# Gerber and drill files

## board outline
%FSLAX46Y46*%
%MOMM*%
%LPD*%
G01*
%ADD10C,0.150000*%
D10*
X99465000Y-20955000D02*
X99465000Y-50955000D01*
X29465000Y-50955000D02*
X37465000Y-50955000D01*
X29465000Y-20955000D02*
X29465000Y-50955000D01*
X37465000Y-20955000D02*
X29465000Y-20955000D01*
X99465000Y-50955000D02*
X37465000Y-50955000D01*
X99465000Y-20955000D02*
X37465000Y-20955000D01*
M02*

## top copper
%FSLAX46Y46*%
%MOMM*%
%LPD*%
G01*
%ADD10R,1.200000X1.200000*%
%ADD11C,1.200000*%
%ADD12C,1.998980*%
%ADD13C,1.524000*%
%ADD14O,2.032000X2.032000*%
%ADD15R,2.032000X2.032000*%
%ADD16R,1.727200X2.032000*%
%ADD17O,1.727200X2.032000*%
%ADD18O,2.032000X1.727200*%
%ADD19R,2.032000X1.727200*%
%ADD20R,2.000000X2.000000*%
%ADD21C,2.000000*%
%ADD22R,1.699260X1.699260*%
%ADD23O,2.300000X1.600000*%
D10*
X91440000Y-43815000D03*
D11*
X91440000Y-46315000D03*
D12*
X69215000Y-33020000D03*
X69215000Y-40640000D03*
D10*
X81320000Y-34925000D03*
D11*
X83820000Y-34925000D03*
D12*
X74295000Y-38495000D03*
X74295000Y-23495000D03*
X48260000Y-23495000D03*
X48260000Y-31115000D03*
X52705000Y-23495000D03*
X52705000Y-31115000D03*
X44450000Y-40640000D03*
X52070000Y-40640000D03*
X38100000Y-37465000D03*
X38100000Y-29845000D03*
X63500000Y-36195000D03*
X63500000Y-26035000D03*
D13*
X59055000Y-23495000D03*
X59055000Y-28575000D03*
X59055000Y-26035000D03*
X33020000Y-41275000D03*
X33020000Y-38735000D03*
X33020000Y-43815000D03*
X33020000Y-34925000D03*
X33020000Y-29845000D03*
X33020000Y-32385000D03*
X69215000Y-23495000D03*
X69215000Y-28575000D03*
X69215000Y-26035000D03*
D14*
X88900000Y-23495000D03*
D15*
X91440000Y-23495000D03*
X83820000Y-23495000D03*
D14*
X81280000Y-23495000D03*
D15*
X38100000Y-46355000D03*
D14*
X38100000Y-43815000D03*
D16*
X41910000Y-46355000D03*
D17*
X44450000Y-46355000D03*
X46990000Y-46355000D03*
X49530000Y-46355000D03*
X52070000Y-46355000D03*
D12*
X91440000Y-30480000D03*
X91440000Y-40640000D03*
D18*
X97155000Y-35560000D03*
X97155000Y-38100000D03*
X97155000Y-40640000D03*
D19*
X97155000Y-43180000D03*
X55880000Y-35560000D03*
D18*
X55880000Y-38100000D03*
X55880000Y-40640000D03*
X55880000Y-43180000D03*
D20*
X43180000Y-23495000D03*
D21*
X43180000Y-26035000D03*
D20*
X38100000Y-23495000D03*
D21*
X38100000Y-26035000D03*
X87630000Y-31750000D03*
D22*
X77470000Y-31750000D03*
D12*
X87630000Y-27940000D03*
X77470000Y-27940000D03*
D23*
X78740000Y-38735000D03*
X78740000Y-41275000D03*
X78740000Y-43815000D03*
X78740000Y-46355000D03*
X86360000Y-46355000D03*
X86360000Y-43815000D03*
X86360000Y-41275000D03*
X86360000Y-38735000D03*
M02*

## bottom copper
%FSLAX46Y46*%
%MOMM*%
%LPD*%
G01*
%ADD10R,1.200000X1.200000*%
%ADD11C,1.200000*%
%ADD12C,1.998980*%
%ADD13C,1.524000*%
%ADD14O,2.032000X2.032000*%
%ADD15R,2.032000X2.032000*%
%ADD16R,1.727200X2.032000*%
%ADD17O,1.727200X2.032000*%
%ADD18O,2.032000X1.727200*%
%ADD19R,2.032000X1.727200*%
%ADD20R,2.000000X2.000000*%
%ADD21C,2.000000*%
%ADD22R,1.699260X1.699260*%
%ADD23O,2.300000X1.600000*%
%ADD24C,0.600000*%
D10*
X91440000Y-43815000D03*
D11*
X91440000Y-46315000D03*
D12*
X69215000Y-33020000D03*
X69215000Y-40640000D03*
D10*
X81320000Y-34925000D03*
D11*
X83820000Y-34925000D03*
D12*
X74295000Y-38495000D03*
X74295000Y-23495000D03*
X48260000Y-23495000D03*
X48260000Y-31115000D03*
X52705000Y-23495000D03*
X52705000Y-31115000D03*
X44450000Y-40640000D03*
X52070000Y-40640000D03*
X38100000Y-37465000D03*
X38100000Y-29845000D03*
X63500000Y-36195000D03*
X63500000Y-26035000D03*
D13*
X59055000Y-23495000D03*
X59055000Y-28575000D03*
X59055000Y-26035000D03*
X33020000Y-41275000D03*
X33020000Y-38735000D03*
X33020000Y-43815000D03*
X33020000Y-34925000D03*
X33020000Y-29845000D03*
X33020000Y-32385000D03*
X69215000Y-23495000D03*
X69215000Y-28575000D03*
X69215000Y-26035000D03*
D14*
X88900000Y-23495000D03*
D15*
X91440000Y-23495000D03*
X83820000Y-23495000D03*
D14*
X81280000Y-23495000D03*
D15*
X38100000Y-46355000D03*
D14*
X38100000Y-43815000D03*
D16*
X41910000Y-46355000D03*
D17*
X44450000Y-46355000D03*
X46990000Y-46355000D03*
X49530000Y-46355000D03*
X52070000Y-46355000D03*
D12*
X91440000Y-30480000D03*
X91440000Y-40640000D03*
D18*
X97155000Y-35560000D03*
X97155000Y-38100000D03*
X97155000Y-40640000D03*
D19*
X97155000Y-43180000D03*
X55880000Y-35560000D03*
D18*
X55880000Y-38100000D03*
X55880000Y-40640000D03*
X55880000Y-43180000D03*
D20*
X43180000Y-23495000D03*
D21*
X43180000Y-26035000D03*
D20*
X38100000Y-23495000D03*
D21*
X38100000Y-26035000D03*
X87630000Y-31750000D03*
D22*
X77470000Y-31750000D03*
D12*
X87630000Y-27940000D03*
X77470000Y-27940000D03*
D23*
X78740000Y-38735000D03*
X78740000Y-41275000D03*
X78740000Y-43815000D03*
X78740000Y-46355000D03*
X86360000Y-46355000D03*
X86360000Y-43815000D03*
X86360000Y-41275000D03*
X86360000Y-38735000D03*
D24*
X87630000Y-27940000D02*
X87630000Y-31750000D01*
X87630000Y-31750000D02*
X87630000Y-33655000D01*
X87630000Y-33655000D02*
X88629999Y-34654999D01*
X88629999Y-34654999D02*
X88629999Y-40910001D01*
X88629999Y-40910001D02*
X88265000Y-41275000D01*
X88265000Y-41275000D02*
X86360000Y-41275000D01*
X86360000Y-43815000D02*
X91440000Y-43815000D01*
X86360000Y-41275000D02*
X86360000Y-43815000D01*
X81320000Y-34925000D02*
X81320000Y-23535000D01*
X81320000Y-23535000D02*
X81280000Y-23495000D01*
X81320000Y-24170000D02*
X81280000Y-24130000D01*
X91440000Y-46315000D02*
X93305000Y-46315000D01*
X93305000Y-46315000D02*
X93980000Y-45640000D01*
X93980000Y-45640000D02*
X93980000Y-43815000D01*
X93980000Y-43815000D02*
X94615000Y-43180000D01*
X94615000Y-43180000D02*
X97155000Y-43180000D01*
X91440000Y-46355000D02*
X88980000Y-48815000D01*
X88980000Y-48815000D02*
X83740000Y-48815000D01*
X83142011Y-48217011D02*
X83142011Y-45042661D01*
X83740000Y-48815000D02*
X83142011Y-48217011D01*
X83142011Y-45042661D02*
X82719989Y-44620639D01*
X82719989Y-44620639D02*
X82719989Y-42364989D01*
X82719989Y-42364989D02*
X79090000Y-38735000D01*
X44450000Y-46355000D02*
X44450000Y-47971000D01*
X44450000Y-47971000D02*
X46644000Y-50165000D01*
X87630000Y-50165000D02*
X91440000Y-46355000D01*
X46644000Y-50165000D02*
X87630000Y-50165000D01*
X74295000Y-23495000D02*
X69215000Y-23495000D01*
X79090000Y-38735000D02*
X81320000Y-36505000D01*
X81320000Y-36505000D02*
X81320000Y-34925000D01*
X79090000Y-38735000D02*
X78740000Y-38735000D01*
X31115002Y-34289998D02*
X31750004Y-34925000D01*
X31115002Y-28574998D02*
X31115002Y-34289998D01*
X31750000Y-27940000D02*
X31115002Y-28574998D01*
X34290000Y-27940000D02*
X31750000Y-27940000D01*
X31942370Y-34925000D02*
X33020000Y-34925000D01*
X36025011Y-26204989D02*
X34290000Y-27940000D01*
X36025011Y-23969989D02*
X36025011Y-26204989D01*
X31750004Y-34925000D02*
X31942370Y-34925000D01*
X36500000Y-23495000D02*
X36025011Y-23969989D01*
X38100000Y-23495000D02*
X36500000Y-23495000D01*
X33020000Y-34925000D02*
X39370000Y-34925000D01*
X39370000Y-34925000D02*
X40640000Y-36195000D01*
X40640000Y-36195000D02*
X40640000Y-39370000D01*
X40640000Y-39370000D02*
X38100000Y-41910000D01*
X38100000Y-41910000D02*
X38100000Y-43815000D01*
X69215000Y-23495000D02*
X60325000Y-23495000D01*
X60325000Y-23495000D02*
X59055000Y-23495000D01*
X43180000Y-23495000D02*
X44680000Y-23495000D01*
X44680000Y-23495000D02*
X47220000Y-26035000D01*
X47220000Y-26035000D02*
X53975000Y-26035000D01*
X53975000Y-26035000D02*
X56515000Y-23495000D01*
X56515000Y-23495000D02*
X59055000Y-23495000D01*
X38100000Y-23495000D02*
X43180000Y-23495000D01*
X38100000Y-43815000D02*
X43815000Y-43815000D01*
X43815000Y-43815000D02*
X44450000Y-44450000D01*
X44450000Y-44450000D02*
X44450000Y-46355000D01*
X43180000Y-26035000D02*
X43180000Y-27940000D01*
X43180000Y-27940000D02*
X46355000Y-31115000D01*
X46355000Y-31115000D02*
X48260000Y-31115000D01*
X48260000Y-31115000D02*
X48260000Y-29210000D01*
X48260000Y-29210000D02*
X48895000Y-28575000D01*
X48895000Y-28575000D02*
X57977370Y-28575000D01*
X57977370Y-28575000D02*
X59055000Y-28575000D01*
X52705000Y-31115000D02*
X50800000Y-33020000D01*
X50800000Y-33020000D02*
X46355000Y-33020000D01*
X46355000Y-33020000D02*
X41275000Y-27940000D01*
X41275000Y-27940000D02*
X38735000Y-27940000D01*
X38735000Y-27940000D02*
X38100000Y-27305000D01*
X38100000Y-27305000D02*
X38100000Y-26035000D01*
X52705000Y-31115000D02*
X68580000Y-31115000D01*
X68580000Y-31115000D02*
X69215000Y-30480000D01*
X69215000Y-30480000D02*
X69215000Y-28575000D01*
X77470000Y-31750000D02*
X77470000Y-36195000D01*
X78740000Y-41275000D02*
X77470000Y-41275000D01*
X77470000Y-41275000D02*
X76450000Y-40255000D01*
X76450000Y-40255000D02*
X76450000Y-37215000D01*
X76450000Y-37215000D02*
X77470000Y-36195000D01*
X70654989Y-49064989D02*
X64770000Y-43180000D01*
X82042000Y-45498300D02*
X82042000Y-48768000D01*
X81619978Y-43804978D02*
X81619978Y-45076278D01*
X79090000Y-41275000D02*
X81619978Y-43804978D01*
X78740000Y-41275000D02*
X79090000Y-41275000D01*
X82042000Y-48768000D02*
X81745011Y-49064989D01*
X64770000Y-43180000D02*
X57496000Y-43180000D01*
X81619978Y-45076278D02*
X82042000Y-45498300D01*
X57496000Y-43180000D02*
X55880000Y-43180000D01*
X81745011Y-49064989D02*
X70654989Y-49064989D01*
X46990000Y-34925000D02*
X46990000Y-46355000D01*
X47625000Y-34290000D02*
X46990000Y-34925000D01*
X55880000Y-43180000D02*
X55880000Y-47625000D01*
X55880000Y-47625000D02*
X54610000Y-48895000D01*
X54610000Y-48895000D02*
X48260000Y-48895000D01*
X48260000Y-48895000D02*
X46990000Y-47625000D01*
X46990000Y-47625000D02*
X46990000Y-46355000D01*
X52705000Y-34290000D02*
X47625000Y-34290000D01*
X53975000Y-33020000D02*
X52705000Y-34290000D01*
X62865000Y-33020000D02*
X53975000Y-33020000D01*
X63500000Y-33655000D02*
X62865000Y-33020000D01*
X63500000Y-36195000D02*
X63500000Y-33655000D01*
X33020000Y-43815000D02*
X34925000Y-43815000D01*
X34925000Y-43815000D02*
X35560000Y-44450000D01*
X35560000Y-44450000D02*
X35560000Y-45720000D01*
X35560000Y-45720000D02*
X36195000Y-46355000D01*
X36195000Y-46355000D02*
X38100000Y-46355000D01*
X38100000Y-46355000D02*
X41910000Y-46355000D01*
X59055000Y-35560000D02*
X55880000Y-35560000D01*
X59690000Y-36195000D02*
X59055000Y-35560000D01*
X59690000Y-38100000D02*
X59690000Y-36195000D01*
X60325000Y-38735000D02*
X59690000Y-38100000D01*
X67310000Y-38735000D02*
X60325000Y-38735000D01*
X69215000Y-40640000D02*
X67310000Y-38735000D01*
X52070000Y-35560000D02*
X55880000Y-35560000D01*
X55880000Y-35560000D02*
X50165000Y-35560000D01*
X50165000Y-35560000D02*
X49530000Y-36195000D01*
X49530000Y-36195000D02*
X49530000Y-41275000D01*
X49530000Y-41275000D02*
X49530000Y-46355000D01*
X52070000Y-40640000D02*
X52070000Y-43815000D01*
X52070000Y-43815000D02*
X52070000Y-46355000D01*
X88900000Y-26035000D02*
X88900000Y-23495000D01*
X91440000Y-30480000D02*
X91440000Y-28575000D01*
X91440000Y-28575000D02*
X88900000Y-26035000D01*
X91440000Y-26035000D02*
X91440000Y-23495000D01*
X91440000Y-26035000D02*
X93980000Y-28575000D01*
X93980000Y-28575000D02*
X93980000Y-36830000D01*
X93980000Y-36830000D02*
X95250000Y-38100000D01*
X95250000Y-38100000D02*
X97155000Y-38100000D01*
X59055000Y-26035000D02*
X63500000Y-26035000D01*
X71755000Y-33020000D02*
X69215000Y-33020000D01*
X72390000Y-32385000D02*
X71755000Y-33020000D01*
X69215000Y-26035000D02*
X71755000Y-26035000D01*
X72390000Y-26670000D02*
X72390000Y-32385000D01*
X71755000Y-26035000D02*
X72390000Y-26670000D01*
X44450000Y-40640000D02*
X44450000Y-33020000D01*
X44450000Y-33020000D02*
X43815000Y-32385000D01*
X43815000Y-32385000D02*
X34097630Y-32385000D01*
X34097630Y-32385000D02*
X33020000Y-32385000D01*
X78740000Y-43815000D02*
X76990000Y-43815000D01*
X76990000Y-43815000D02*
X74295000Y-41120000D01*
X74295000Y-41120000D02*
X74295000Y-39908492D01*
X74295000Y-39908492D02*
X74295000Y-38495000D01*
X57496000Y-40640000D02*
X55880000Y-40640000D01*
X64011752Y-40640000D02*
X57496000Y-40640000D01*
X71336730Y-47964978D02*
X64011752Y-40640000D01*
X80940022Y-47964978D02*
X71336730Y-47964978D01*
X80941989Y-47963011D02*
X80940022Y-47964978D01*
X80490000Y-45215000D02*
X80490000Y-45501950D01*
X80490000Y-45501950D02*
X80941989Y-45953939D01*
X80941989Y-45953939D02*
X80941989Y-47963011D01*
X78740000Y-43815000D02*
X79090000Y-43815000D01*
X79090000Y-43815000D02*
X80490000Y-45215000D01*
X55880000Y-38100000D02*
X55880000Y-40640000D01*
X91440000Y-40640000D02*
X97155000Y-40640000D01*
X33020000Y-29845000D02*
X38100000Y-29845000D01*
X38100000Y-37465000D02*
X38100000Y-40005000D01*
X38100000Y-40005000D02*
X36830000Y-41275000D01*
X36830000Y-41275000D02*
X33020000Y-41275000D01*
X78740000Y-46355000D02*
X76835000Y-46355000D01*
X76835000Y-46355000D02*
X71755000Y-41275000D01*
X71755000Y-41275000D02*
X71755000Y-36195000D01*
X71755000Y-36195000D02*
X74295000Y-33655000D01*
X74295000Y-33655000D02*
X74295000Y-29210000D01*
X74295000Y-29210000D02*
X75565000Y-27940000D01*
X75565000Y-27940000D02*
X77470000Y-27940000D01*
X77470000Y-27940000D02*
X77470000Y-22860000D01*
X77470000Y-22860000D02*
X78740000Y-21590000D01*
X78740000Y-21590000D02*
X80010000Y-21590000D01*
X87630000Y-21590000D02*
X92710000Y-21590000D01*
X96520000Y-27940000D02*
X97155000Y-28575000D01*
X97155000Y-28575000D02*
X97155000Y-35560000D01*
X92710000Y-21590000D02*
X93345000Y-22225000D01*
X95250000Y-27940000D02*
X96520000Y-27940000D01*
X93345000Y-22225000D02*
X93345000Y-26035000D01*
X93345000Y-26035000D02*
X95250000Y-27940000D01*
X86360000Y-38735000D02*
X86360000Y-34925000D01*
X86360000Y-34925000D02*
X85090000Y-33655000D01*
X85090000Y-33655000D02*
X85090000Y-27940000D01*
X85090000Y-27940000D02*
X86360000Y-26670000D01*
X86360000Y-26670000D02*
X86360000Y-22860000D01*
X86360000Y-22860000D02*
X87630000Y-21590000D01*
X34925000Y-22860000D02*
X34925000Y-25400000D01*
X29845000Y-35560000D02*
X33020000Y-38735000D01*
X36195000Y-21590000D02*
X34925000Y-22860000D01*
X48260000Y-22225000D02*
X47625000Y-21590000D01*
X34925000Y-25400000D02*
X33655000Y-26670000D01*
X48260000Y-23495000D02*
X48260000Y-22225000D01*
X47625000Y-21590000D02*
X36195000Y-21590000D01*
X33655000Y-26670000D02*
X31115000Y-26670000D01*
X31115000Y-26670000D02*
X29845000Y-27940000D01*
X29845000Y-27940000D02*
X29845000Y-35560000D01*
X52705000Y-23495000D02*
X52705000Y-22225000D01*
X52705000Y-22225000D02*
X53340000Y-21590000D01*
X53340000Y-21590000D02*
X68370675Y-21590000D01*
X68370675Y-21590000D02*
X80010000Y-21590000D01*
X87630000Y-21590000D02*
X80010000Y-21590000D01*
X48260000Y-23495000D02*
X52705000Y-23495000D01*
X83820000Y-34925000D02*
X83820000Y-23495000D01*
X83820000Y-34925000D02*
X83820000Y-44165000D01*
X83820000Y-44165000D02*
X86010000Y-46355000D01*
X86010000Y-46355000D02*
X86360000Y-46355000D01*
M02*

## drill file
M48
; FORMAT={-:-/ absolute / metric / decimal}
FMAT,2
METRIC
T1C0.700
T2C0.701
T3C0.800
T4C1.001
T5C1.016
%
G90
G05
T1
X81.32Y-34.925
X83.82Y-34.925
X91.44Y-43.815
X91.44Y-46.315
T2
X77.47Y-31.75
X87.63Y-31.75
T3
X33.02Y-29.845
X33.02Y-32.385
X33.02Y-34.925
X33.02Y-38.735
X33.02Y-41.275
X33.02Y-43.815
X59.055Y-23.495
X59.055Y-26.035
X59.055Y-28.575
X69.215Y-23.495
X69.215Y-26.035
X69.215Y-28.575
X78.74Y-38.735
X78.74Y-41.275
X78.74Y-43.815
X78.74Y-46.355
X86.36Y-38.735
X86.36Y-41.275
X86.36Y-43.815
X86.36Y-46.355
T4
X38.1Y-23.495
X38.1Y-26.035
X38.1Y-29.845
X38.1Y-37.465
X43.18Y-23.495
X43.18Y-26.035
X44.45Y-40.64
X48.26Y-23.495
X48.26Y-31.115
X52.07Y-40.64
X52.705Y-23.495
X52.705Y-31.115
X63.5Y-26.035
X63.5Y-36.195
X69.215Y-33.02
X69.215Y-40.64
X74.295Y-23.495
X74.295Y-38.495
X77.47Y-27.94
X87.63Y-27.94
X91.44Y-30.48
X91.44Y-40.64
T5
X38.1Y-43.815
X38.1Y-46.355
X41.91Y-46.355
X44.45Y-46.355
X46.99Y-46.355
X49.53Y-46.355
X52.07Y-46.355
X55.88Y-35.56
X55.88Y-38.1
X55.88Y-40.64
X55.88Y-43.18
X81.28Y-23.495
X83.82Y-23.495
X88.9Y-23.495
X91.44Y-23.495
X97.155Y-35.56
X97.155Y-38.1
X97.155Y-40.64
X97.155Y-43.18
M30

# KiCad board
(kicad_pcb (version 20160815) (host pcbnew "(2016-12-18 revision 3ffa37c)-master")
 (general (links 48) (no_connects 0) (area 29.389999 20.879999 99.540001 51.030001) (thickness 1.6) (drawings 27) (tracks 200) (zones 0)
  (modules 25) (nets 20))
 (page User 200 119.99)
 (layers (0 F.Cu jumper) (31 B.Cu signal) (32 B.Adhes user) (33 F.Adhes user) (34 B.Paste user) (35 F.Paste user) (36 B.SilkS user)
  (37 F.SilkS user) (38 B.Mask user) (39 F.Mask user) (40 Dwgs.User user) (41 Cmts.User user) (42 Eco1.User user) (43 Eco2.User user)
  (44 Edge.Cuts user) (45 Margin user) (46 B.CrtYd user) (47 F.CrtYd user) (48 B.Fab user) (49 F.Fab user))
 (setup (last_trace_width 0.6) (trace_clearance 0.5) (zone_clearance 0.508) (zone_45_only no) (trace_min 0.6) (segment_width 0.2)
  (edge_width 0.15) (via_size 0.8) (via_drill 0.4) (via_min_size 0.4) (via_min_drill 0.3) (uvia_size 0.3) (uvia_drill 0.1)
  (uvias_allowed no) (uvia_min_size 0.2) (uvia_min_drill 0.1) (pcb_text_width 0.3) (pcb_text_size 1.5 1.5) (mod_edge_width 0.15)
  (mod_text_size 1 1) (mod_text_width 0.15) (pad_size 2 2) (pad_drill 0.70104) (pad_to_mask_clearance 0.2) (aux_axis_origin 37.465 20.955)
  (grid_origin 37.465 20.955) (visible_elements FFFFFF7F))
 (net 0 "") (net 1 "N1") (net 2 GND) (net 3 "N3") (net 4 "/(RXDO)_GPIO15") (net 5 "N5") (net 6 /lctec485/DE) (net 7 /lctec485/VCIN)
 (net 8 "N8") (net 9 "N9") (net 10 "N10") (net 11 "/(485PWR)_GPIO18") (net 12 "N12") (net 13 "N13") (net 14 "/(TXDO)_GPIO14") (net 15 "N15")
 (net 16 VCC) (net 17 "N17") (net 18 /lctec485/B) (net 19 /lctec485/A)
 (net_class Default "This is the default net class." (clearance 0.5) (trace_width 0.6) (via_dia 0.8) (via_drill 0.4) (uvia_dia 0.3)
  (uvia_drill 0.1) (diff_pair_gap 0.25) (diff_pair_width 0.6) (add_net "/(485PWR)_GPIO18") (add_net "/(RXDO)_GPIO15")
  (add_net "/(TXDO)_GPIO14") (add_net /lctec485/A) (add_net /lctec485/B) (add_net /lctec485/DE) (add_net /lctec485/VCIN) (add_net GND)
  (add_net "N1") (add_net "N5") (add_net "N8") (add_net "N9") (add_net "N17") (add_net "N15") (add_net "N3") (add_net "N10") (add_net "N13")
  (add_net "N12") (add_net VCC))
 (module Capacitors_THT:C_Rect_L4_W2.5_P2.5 (layer F.Cu) (at 91.44 43.815 270)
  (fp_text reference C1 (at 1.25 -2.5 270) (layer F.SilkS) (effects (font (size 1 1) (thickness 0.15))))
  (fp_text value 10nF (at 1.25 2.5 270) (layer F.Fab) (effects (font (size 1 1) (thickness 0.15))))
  (pad 1 thru_hole rect (at 0 0 270) (size 1.2 1.2) (drill 0.7) (layers *.Cu *.Mask) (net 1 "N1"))
  (pad 2 thru_hole circle (at 2.5 0 270) (size 1.2 1.2) (drill 0.7) (layers *.Cu *.Mask) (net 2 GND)))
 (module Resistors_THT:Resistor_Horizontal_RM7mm (layer F.Cu) (at 69.215 33.02 270)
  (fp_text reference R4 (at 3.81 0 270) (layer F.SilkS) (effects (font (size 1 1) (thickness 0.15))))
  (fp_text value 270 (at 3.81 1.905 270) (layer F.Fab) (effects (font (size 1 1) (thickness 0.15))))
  (pad 1 thru_hole circle (at 0 0 270) (size 1.99898 1.99898) (drill 1.00076) (layers *.Cu *.SilkS *.Mask) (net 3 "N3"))
  (pad 2 thru_hole circle (at 7.62 0 270) (size 1.99898 1.99898) (drill 1.00076) (layers *.Cu *.SilkS *.Mask) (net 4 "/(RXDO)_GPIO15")))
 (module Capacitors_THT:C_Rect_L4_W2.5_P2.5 (layer F.Cu) (at 81.32 34.925)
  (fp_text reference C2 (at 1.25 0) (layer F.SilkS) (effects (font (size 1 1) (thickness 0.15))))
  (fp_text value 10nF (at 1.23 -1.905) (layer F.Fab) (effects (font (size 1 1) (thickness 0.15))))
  (pad 1 thru_hole rect (at 0 0) (size 1.2 1.2) (drill 0.7) (layers *.Cu *.Mask) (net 2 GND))
  (pad 2 thru_hole circle (at 2.5 0) (size 1.2 1.2) (drill 0.7) (layers *.Cu *.Mask) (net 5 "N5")))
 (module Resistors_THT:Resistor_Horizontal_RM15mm (layer F.Cu) (at 74.295 38.495 90)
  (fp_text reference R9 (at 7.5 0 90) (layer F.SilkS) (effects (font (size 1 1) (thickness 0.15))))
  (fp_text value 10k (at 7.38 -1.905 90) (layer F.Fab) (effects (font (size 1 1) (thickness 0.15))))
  (pad 1 thru_hole circle (at 0 0 90) (size 1.99898 1.99898) (drill 1.00076) (layers *.Cu *.SilkS *.Mask) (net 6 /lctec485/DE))
  (pad 2 thru_hole circle (at 15 0 90) (size 1.99898 1.99898) (drill 1.00076) (layers *.Cu *.SilkS *.Mask) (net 2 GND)))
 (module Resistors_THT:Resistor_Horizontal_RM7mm (layer F.Cu) (at 48.26 31.115 90)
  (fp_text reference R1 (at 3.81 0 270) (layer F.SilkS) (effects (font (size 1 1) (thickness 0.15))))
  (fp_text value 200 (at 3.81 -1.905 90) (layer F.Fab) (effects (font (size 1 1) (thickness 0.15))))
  (pad 2 thru_hole circle (at 7.62 0 90) (size 1.99898 1.99898) (drill 1.00076) (layers *.Cu *.SilkS *.Mask) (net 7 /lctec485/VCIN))
  (pad 1 thru_hole circle (at 0 0 90) (size 1.99898 1.99898) (drill 1.00076) (layers *.Cu *.SilkS *.Mask) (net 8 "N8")))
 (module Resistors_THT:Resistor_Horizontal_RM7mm (layer F.Cu) (at 52.705 31.115 90)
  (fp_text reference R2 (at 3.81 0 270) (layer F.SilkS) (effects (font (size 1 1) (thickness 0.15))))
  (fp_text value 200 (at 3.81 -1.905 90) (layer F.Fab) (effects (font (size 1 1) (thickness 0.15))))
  (pad 2 thru_hole circle (at 7.62 0 90) (size 1.99898 1.99898) (drill 1.00076) (layers *.Cu *.SilkS *.Mask) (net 7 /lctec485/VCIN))
  (pad 1 thru_hole circle (at 0 0 90) (size 1.99898 1.99898) (drill 1.00076) (layers *.Cu *.SilkS *.Mask) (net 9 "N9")))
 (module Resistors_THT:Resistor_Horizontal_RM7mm (layer F.Cu) (at 52.07 40.64 180)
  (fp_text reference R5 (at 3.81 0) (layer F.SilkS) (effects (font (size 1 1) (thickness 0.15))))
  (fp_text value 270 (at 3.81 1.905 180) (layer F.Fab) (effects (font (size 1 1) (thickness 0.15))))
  (pad 2 thru_hole circle (at 7.62 0 180) (size 1.99898 1.99898) (drill 1.00076) (layers *.Cu *.SilkS *.Mask) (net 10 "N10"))
  (pad 1 thru_hole circle (at 0 0 180) (size 1.99898 1.99898) (drill 1.00076) (layers *.Cu *.SilkS *.Mask) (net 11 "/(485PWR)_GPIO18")))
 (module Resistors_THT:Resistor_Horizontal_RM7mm (layer F.Cu) (at 38.1 29.845 270)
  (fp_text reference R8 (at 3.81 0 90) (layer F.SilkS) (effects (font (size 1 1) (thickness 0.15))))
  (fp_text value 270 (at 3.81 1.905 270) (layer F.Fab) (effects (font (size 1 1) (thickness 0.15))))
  (pad 2 thru_hole circle (at 7.62 0 270) (size 1.99898 1.99898) (drill 1.00076) (layers *.Cu *.SilkS *.Mask) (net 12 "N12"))
  (pad 1 thru_hole circle (at 0 0 270) (size 1.99898 1.99898) (drill 1.00076) (layers *.Cu *.SilkS *.Mask) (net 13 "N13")))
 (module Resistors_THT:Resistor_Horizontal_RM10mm (layer F.Cu) (at 63.5 26.035 270)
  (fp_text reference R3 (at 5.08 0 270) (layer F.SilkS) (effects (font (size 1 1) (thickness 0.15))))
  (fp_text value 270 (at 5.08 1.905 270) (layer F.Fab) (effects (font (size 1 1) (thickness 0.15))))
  (pad 2 thru_hole circle (at 10.16 0 270) (size 1.99898 1.99898) (drill 1.00076) (layers *.Cu *.SilkS *.Mask) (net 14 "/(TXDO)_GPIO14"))
  (pad 1 thru_hole circle (at 0 0 270) (size 1.99898 1.99898) (drill 1.00076) (layers *.Cu *.SilkS *.Mask) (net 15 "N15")))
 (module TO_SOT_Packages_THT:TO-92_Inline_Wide (layer F.Cu) (at 59.055 23.495 270)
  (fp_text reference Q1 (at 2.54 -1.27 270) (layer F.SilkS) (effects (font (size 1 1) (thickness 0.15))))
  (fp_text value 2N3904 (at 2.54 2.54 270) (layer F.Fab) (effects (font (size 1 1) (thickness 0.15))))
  (pad 1 thru_hole circle (at 0 0) (size 1.524 1.524) (drill 0.8) (layers *.Cu *.Mask) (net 2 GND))
  (pad 3 thru_hole circle (at 5.08 0) (size 1.524 1.524) (drill 0.8) (layers *.Cu *.Mask) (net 8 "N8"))
  (pad 2 thru_hole circle (at 2.54 0) (size 1.524 1.524) (drill 0.8) (layers *.Cu *.Mask) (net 15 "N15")))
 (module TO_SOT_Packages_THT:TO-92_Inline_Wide (layer F.Cu) (at 33.02 43.815 90)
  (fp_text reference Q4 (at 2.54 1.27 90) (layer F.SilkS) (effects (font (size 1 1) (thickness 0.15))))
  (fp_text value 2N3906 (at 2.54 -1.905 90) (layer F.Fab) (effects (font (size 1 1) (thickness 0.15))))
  (pad 2 thru_hole circle (at 2.54 0 180) (size 1.524 1.524) (drill 0.8) (layers *.Cu *.Mask) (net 12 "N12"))
  (pad 3 thru_hole circle (at 5.08 0 180) (size 1.524 1.524) (drill 0.8) (layers *.Cu *.Mask) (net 7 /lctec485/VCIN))
  (pad 1 thru_hole circle (at 0 0 180) (size 1.524 1.524) (drill 0.8) (layers *.Cu *.Mask) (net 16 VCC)))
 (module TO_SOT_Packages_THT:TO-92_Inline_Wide (layer F.Cu) (at 33.02 34.925 90)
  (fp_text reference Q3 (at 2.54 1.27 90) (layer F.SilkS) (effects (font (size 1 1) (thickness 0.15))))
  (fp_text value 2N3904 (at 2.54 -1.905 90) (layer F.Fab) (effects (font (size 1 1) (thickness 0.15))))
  (pad 1 thru_hole circle (at 0 0 180) (size 1.524 1.524) (drill 0.8) (layers *.Cu *.Mask) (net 2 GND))
  (pad 3 thru_hole circle (at 5.08 0 180) (size 1.524 1.524) (drill 0.8) (layers *.Cu *.Mask) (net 13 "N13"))
  (pad 2 thru_hole circle (at 2.54 0 180) (size 1.524 1.524) (drill 0.8) (layers *.Cu *.Mask) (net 10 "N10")))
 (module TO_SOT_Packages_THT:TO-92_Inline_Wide (layer F.Cu) (at 69.215 23.495 270)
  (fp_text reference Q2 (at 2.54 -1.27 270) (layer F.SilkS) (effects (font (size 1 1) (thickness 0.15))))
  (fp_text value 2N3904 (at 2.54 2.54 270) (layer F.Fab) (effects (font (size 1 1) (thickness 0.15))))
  (pad 1 thru_hole circle (at 0 0) (size 1.524 1.524) (drill 0.8) (layers *.Cu *.Mask) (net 2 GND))
  (pad 3 thru_hole circle (at 5.08 0) (size 1.524 1.524) (drill 0.8) (layers *.Cu *.Mask) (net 9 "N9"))
  (pad 2 thru_hole circle (at 2.54 0) (size 1.524 1.524) (drill 0.8) (layers *.Cu *.Mask) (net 3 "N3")))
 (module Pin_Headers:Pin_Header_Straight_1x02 (layer F.Cu) (at 91.44 23.495 270)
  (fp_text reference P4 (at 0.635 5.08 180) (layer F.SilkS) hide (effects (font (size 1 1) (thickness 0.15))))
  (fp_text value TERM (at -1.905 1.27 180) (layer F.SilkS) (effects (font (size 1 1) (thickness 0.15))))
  (pad 2 thru_hole oval (at 0 2.54 270) (size 2.032 2.032) (drill 1.016) (layers *.Cu *.Mask) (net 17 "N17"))
  (pad 1 thru_hole rect (at 0 0 270) (size 2.032 2.032) (drill 1.016) (layers *.Cu *.Mask) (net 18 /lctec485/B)))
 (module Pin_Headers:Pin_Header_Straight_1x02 (layer F.Cu) (at 83.82 23.495 270)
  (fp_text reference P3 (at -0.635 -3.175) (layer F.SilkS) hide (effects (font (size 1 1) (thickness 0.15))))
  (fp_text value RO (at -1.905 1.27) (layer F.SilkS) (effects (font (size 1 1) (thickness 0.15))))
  (pad 1 thru_hole rect (at 0 0 270) (size 2.032 2.032) (drill 1.016) (layers *.Cu *.Mask) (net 5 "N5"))
  (pad 2 thru_hole oval (at 0 2.54 270) (size 2.032 2.032) (drill 1.016) (layers *.Cu *.Mask) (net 2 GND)))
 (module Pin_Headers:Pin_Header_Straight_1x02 (layer F.Cu) (at 38.1 46.355 180)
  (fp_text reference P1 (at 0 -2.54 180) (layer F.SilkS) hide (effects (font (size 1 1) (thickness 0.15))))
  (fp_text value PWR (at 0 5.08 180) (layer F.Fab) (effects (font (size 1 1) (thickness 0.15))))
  (pad 1 thru_hole rect (at 0 0 180) (size 2.032 2.032) (drill 1.016) (layers *.Cu *.Mask) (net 16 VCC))
  (pad 2 thru_hole oval (at 0 2.54 180) (size 2.032 2.032) (drill 1.016) (layers *.Cu *.Mask) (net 2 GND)))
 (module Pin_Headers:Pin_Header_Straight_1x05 (layer F.Cu) (at 41.91 46.355 90)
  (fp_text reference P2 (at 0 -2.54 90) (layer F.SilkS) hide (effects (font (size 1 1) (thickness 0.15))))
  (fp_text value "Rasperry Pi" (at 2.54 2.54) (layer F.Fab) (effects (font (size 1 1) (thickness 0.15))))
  (pad 1 thru_hole rect (at 0 0 90) (size 2.032 1.7272) (drill 1.016) (layers *.Cu *.Mask) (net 16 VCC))
  (pad 2 thru_hole oval (at 0 2.54 90) (size 2.032 1.7272) (drill 1.016) (layers *.Cu *.Mask) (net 2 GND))
  (pad 3 thru_hole oval (at 0 5.08 90) (size 2.032 1.7272) (drill 1.016) (layers *.Cu *.Mask) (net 14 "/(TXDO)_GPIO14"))
  (pad 4 thru_hole oval (at 0 7.62 90) (size 2.032 1.7272) (drill 1.016) (layers *.Cu *.Mask) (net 4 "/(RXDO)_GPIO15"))
  (pad 5 thru_hole oval (at 0 10.16 90) (size 2.032 1.7272) (drill 1.016) (layers *.Cu *.Mask) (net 11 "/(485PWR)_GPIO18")))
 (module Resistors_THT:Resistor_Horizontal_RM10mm (layer F.Cu) (at 91.44 30.48 270)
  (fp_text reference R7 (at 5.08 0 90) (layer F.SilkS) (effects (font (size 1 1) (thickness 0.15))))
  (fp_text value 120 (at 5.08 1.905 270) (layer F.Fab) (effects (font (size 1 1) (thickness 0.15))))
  (pad 1 thru_hole circle (at 0 0 270) (size 1.99898 1.99898) (drill 1.00076) (layers *.Cu *.SilkS *.Mask) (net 17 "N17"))
  (pad 2 thru_hole circle (at 10.16 0 270) (size 1.99898 1.99898) (drill 1.00076) (layers *.Cu *.SilkS *.Mask) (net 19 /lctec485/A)))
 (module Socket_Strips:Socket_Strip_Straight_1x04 (layer F.Cu) (at 97.155 43.18 90)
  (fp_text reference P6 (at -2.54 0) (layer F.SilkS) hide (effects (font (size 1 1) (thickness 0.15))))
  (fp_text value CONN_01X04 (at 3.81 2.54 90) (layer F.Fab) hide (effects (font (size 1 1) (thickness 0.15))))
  (pad 4 thru_hole oval (at 7.62 0 90) (size 1.7272 2.032) (drill 1.016) (layers *.Cu *.Mask) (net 7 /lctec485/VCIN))
  (pad 3 thru_hole oval (at 5.08 0 90) (size 1.7272 2.032) (drill 1.016) (layers *.Cu *.Mask) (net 18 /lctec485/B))
  (pad 2 thru_hole oval (at 2.54 0 90) (size 1.7272 2.032) (drill 1.016) (layers *.Cu *.Mask) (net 19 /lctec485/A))
  (pad 1 thru_hole rect (at 0 0 90) (size 1.7272 2.032) (drill 1.016) (layers *.Cu *.Mask) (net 2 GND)))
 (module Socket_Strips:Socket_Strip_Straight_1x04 (layer F.Cu) (at 55.88 35.56 270)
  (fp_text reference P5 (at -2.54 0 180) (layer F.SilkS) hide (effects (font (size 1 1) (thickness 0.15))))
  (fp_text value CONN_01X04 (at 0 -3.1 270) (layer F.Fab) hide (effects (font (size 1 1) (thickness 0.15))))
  (pad 1 thru_hole rect (at 0 0 270) (size 1.7272 2.032) (drill 1.016) (layers *.Cu *.Mask) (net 4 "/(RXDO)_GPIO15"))
  (pad 2 thru_hole oval (at 2.54 0 270) (size 1.7272 2.032) (drill 1.016) (layers *.Cu *.Mask) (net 6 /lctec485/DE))
  (pad 3 thru_hole oval (at 5.08 0 270) (size 1.7272 2.032) (drill 1.016) (layers *.Cu *.Mask) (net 6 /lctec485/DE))
  (pad 4 thru_hole oval (at 7.62 0 270) (size 1.7272 2.032) (drill 1.016) (layers *.Cu *.Mask) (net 14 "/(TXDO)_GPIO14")))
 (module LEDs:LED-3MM (layer F.Cu) (at 43.18 23.495 270)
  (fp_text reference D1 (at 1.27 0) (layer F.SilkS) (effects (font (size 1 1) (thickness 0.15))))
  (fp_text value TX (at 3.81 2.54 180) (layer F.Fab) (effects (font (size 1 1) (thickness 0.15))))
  (pad 1 thru_hole rect (at 0 0) (size 2 2) (drill 1.00076) (layers *.Cu *.Mask) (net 2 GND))
  (pad 2 thru_hole circle (at 2.54 0 270) (size 2 2) (drill 1.00076) (layers *.Cu *.Mask) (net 8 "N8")))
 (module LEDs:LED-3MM (layer F.Cu) (at 38.1 23.495 270)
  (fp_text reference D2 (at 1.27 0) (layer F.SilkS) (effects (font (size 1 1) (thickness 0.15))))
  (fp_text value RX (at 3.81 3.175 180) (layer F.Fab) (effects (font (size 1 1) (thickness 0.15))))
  (pad 1 thru_hole rect (at 0 0) (size 2 2) (drill 1.00076) (layers *.Cu *.Mask) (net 2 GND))
  (pad 2 thru_hole circle (at 2.54 0 270) (size 2 2) (drill 1.00076) (layers *.Cu *.Mask) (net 9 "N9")))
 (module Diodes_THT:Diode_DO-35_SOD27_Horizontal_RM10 (layer F.Cu) (at 77.46948 31.75254)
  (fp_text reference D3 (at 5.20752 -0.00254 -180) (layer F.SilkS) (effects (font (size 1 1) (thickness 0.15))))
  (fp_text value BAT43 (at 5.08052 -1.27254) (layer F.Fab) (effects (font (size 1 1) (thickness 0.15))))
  (pad 2 thru_hole circle (at 10.16052 -0.00254 180) (size 2 2) (drill 0.70104) (layers *.Cu *.Mask) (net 1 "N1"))
  (pad 1 thru_hole rect (at 0.00052 -0.00254 180) (size 1.69926 1.69926) (drill 0.70104) (layers *.Cu *.Mask) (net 14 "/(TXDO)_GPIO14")))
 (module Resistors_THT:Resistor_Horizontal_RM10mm (layer F.Cu) (at 87.63 27.94 180)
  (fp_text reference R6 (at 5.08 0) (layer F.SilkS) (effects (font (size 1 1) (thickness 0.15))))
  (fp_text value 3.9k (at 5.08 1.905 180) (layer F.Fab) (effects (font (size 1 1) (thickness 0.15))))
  (pad 1 thru_hole circle (at 0 0 180) (size 1.99898 1.99898) (drill 1.00076) (layers *.Cu *.SilkS *.Mask) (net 1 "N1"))
  (pad 2 thru_hole circle (at 10.16 0 180) (size 1.99898 1.99898) (drill 1.00076) (layers *.Cu *.SilkS *.Mask) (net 7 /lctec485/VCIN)))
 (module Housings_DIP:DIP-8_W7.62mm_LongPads (layer F.Cu) (at 78.74 38.735)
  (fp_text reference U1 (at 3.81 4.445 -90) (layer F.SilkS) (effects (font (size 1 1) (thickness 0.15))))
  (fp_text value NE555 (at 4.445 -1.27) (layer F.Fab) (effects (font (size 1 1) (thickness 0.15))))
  (pad 1 thru_hole oval (at 0 0) (size 2.3 1.6) (drill 0.8) (layers *.Cu *.Mask) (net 2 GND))
  (pad 2 thru_hole oval (at 0 2.54) (size 2.3 1.6) (drill 0.8) (layers *.Cu *.Mask) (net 14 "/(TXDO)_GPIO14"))
  (pad 3 thru_hole oval (at 0 5.08) (size 2.3 1.6) (drill 0.8) (layers *.Cu *.Mask) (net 6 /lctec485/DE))
  (pad 4 thru_hole oval (at 0 7.62) (size 2.3 1.6) (drill 0.8) (layers *.Cu *.Mask) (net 7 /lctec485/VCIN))
  (pad 5 thru_hole oval (at 7.62 7.62) (size 2.3 1.6) (drill 0.8) (layers *.Cu *.Mask) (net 5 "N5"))
  (pad 6 thru_hole oval (at 7.62 5.08) (size 2.3 1.6) (drill 0.8) (layers *.Cu *.Mask) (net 1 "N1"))
  (pad 7 thru_hole oval (at 7.62 2.54) (size 2.3 1.6) (drill 0.8) (layers *.Cu *.Mask) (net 1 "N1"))
  (pad 8 thru_hole oval (at 7.62 0) (size 2.3 1.6) (drill 0.8) (layers *.Cu *.Mask) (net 7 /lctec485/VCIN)))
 (gr_line (start 99.465 20.955) (end 99.465 50.955) (layer Edge.Cuts) (width 0.15))
 (gr_line (start 29.465 50.955) (end 37.465 50.955) (layer Edge.Cuts) (width 0.15))
 (gr_line (start 29.465 20.955) (end 29.465 50.955) (layer Edge.Cuts) (width 0.15))
 (gr_line (start 37.465 20.955) (end 29.465 20.955) (layer Edge.Cuts) (width 0.15))
 (gr_line (start 99.465 50.955) (end 37.465 50.955) (layer Edge.Cuts) (width 0.15))
 (gr_line (start 99.465 20.955) (end 37.465 20.955) (layer Edge.Cuts) (width 0.15))
 (segment (start 87.63 27.94) (end 87.63 31.75) (width 0.6) (layer B.Cu) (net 1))
 (segment (start 87.63 31.75) (end 87.63 33.655) (width 0.6) (layer B.Cu) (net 1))
 (segment (start 87.63 33.655) (end 88.629999 34.654999) (width 0.6) (layer B.Cu) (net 1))
 (segment (start 88.629999 34.654999) (end 88.629999 40.910001) (width 0.6) (layer B.Cu) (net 1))
 (segment (start 88.629999 40.910001) (end 88.265 41.275) (width 0.6) (layer B.Cu) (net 1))
 (segment (start 88.265 41.275) (end 86.36 41.275) (width 0.6) (layer B.Cu) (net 1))
 (segment (start 86.36 43.815) (end 91.44 43.815) (width 0.6) (layer B.Cu) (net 1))
 (segment (start 86.36 41.275) (end 86.36 43.815) (width 0.6) (layer B.Cu) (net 1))
 (segment (start 81.32 34.925) (end 81.32 23.535) (width 0.6) (layer B.Cu) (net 2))
 (segment (start 81.32 23.535) (end 81.28 23.495) (width 0.6) (layer B.Cu) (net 2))
 (segment (start 81.32 24.17) (end 81.28 24.13) (width 0.6) (layer B.Cu) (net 2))
 (segment (start 91.44 46.315) (end 93.305 46.315) (width 0.6) (layer B.Cu) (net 2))
 (segment (start 93.305 46.315) (end 93.98 45.64) (width 0.6) (layer B.Cu) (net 2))
 (segment (start 93.98 45.64) (end 93.98 43.815) (width 0.6) (layer B.Cu) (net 2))
 (segment (start 93.98 43.815) (end 94.615 43.18) (width 0.6) (layer B.Cu) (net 2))
 (segment (start 94.615 43.18) (end 97.155 43.18) (width 0.6) (layer B.Cu) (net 2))
 (segment (start 91.44 46.355) (end 88.98 48.815) (width 0.6) (layer B.Cu) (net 2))
 (segment (start 88.98 48.815) (end 83.74 48.815) (width 0.6) (layer B.Cu) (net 2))
 (segment (start 83.142011 48.217011) (end 83.142011 45.042661) (width 0.6) (layer B.Cu) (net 2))
 (segment (start 83.74 48.815) (end 83.142011 48.217011) (width 0.6) (layer B.Cu) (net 2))
 (segment (start 83.142011 45.042661) (end 82.719989 44.620639) (width 0.6) (layer B.Cu) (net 2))
 (segment (start 82.719989 44.620639) (end 82.719989 42.364989) (width 0.6) (layer B.Cu) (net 2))
 (segment (start 82.719989 42.364989) (end 79.09 38.735) (width 0.6) (layer B.Cu) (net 2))
 (segment (start 44.45 46.355) (end 44.45 47.971) (width 0.6) (layer B.Cu) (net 2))
 (segment (start 44.45 47.971) (end 46.644 50.165) (width 0.6) (layer B.Cu) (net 2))
 (segment (start 87.63 50.165) (end 91.44 46.355) (width 0.6) (layer B.Cu) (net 2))
 (segment (start 46.644 50.165) (end 87.63 50.165) (width 0.6) (layer B.Cu) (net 2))
 (segment (start 74.295 23.495) (end 69.215 23.495) (width 0.6) (layer B.Cu) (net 2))
 (segment (start 79.09 38.735) (end 81.32 36.505) (width 0.6) (layer B.Cu) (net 2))
 (segment (start 81.32 36.505) (end 81.32 34.925) (width 0.6) (layer B.Cu) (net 2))
 (segment (start 79.09 38.735) (end 78.74 38.735) (width 0.6) (layer B.Cu) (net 2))
 (segment (start 31.115002 34.289998) (end 31.750004 34.925) (width 0.6) (layer B.Cu) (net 2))
 (segment (start 31.115002 28.574998) (end 31.115002 34.289998) (width 0.6) (layer B.Cu) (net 2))
 (segment (start 31.75 27.94) (end 31.115002 28.574998) (width 0.6) (layer B.Cu) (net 2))
 (segment (start 34.29 27.94) (end 31.75 27.94) (width 0.6) (layer B.Cu) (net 2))
 (segment (start 31.94237 34.925) (end 33.02 34.925) (width 0.6) (layer B.Cu) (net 2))
 (segment (start 36.025011 26.204989) (end 34.29 27.94) (width 0.6) (layer B.Cu) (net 2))
 (segment (start 36.025011 23.969989) (end 36.025011 26.204989) (width 0.6) (layer B.Cu) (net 2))
 (segment (start 31.750004 34.925) (end 31.94237 34.925) (width 0.6) (layer B.Cu) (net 2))
 (segment (start 36.5 23.495) (end 36.025011 23.969989) (width 0.6) (layer B.Cu) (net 2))
 (segment (start 38.1 23.495) (end 36.5 23.495) (width 0.6) (layer B.Cu) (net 2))
 (segment (start 33.02 34.925) (end 39.37 34.925) (width 0.6) (layer B.Cu) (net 2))
 (segment (start 39.37 34.925) (end 40.64 36.195) (width 0.6) (layer B.Cu) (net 2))
 (segment (start 40.64 36.195) (end 40.64 39.37) (width 0.6) (layer B.Cu) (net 2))
 (segment (start 40.64 39.37) (end 38.1 41.91) (width 0.6) (layer B.Cu) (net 2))
 (segment (start 38.1 41.91) (end 38.1 43.815) (width 0.6) (layer B.Cu) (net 2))
 (segment (start 69.215 23.495) (end 60.325 23.495) (width 0.6) (layer B.Cu) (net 2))
 (segment (start 60.325 23.495) (end 59.055 23.495) (width 0.6) (layer B.Cu) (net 2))
 (segment (start 43.18 23.495) (end 44.68 23.495) (width 0.6) (layer B.Cu) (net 2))
 (segment (start 44.68 23.495) (end 47.22 26.035) (width 0.6) (layer B.Cu) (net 2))
 (segment (start 47.22 26.035) (end 53.975 26.035) (width 0.6) (layer B.Cu) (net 2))
 (segment (start 53.975 26.035) (end 56.515 23.495) (width 0.6) (layer B.Cu) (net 2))
 (segment (start 56.515 23.495) (end 59.055 23.495) (width 0.6) (layer B.Cu) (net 2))
 (segment (start 38.1 23.495) (end 43.18 23.495) (width 0.6) (layer B.Cu) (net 2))
 (segment (start 38.1 43.815) (end 43.815 43.815) (width 0.6) (layer B.Cu) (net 2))
 (segment (start 43.815 43.815) (end 44.45 44.45) (width 0.6) (layer B.Cu) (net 2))
 (segment (start 44.45 44.45) (end 44.45 46.355) (width 0.6) (layer B.Cu) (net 2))
 (segment (start 43.18 26.035) (end 43.18 27.94) (width 0.6) (layer B.Cu) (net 8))
 (segment (start 43.18 27.94) (end 46.355 31.115) (width 0.6) (layer B.Cu) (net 8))
 (segment (start 46.355 31.115) (end 48.26 31.115) (width 0.6) (layer B.Cu) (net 8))
 (segment (start 48.26 31.115) (end 48.26 29.21) (width 0.6) (layer B.Cu) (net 8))
 (segment (start 48.26 29.21) (end 48.895 28.575) (width 0.6) (layer B.Cu) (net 8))
 (segment (start 48.895 28.575) (end 57.97737 28.575) (width 0.6) (layer B.Cu) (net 8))
 (segment (start 57.97737 28.575) (end 59.055 28.575) (width 0.6) (layer B.Cu) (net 8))
 (segment (start 52.705 31.115) (end 50.8 33.02) (width 0.6) (layer B.Cu) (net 9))
 (segment (start 50.8 33.02) (end 46.355 33.02) (width 0.6) (layer B.Cu) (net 9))
 (segment (start 46.355 33.02) (end 41.275 27.94) (width 0.6) (layer B.Cu) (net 9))
 (segment (start 41.275 27.94) (end 38.735 27.94) (width 0.6) (layer B.Cu) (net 9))
 (segment (start 38.735 27.94) (end 38.1 27.305) (width 0.6) (layer B.Cu) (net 9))
 (segment (start 38.1 27.305) (end 38.1 26.035) (width 0.6) (layer B.Cu) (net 9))
 (segment (start 52.705 31.115) (end 68.58 31.115) (width 0.6) (layer B.Cu) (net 9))
 (segment (start 68.58 31.115) (end 69.215 30.48) (width 0.6) (layer B.Cu) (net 9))
 (segment (start 69.215 30.48) (end 69.215 28.575) (width 0.6) (layer B.Cu) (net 9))
 (segment (start 77.47 31.75) (end 77.47 36.195) (width 0.6) (layer B.Cu) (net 14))
 (segment (start 78.74 41.275) (end 77.47 41.275) (width 0.6) (layer B.Cu) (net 14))
 (segment (start 77.47 41.275) (end 76.45 40.255) (width 0.6) (layer B.Cu) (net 14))
 (segment (start 76.45 40.255) (end 76.45 37.215) (width 0.6) (layer B.Cu) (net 14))
 (segment (start 76.45 37.215) (end 77.47 36.195) (width 0.6) (layer B.Cu) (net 14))
 (segment (start 70.654989 49.064989) (end 64.77 43.18) (width 0.6) (layer B.Cu) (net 14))
 (segment (start 82.042 45.4983) (end 82.042 48.768) (width 0.6) (layer B.Cu) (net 14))
 (segment (start 81.619978 43.804978) (end 81.619978 45.076278) (width 0.6) (layer B.Cu) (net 14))
 (segment (start 79.09 41.275) (end 81.619978 43.804978) (width 0.6) (layer B.Cu) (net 14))
 (segment (start 78.74 41.275) (end 79.09 41.275) (width 0.6) (layer B.Cu) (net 14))
 (segment (start 82.042 48.768) (end 81.745011 49.064989) (width 0.6) (layer B.Cu) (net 14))
 (segment (start 64.77 43.18) (end 57.496 43.18) (width 0.6) (layer B.Cu) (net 14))
 (segment (start 81.619978 45.076278) (end 82.042 45.4983) (width 0.6) (layer B.Cu) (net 14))
 (segment (start 57.496 43.18) (end 55.88 43.18) (width 0.6) (layer B.Cu) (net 14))
 (segment (start 81.745011 49.064989) (end 70.654989 49.064989) (width 0.6) (layer B.Cu) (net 14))
 (segment (start 46.99 34.925) (end 46.99 46.355) (width 0.6) (layer B.Cu) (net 14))
 (segment (start 47.625 34.29) (end 46.99 34.925) (width 0.6) (layer B.Cu) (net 14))
 (segment (start 55.88 43.18) (end 55.88 47.625) (width 0.6) (layer B.Cu) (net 14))
 (segment (start 55.88 47.625) (end 54.61 48.895) (width 0.6) (layer B.Cu) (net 14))
 (segment (start 54.61 48.895) (end 48.26 48.895) (width 0.6) (layer B.Cu) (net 14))
 (segment (start 48.26 48.895) (end 46.99 47.625) (width 0.6) (layer B.Cu) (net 14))
 (segment (start 46.99 47.625) (end 46.99 46.355) (width 0.6) (layer B.Cu) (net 14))
 (segment (start 52.705 34.29) (end 47.625 34.29) (width 0.6) (layer B.Cu) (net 14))
 (segment (start 53.975 33.02) (end 52.705 34.29) (width 0.6) (layer B.Cu) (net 14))
 (segment (start 62.865 33.02) (end 53.975 33.02) (width 0.6) (layer B.Cu) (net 14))
 (segment (start 63.5 33.655) (end 62.865 33.02) (width 0.6) (layer B.Cu) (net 14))
 (segment (start 63.5 36.195) (end 63.5 33.655) (width 0.6) (layer B.Cu) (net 14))
 (segment (start 33.02 43.815) (end 34.925 43.815) (width 0.6) (layer B.Cu) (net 16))
 (segment (start 34.925 43.815) (end 35.56 44.45) (width 0.6) (layer B.Cu) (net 16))
 (segment (start 35.56 44.45) (end 35.56 45.72) (width 0.6) (layer B.Cu) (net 16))
 (segment (start 35.56 45.72) (end 36.195 46.355) (width 0.6) (layer B.Cu) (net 16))
 (segment (start 36.195 46.355) (end 38.1 46.355) (width 0.6) (layer B.Cu) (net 16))
 (segment (start 38.1 46.355) (end 41.91 46.355) (width 0.6) (layer B.Cu) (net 16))
 (segment (start 59.055 35.56) (end 55.88 35.56) (width 0.6) (layer B.Cu) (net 4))
 (segment (start 59.69 36.195) (end 59.055 35.56) (width 0.6) (layer B.Cu) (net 4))
 (segment (start 59.69 38.1) (end 59.69 36.195) (width 0.6) (layer B.Cu) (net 4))
 (segment (start 60.325 38.735) (end 59.69 38.1) (width 0.6) (layer B.Cu) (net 4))
 (segment (start 67.31 38.735) (end 60.325 38.735) (width 0.6) (layer B.Cu) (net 4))
 (segment (start 69.215 40.64) (end 67.31 38.735) (width 0.6) (layer B.Cu) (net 4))
 (segment (start 52.07 35.56) (end 55.88 35.56) (width 0.6) (layer B.Cu) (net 4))
 (segment (start 55.88 35.56) (end 50.165 35.56) (width 0.6) (layer B.Cu) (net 4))
 (segment (start 50.165 35.56) (end 49.53 36.195) (width 0.6) (layer B.Cu) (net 4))
 (segment (start 49.53 36.195) (end 49.53 41.275) (width 0.6) (layer B.Cu) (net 4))
 (segment (start 49.53 41.275) (end 49.53 46.355) (width 0.6) (layer B.Cu) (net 4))
 (segment (start 52.07 40.64) (end 52.07 43.815) (width 0.6) (layer B.Cu) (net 11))
 (segment (start 52.07 43.815) (end 52.07 46.355) (width 0.6) (layer B.Cu) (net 11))
 (segment (start 88.9 26.035) (end 88.9 23.495) (width 0.6) (layer B.Cu) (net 17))
 (segment (start 91.44 30.48) (end 91.44 28.575) (width 0.6) (layer B.Cu) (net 17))
 (segment (start 91.44 28.575) (end 88.9 26.035) (width 0.6) (layer B.Cu) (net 17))
 (segment (start 91.44 26.035) (end 91.44 23.495) (width 0.6) (layer B.Cu) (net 18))
 (segment (start 91.44 26.035) (end 93.98 28.575) (width 0.6) (layer B.Cu) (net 18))
 (segment (start 93.98 28.575) (end 93.98 36.83) (width 0.6) (layer B.Cu) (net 18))
 (segment (start 93.98 36.83) (end 95.25 38.1) (width 0.6) (layer B.Cu) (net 18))
 (segment (start 95.25 38.1) (end 97.155 38.1) (width 0.6) (layer B.Cu) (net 18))
 (segment (start 59.055 26.035) (end 63.5 26.035) (width 0.6) (layer B.Cu) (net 15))
 (segment (start 71.755 33.02) (end 69.215 33.02) (width 0.6) (layer B.Cu) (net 3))
 (segment (start 72.39 32.385) (end 71.755 33.02) (width 0.6) (layer B.Cu) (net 3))
 (segment (start 69.215 26.035) (end 71.755 26.035) (width 0.6) (layer B.Cu) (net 3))
 (segment (start 72.39 26.67) (end 72.39 32.385) (width 0.6) (layer B.Cu) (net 3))
 (segment (start 71.755 26.035) (end 72.39 26.67) (width 0.6) (layer B.Cu) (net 3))
 (segment (start 44.45 40.64) (end 44.45 33.02) (width 0.6) (layer B.Cu) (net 10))
 (segment (start 44.45 33.02) (end 43.815 32.385) (width 0.6) (layer B.Cu) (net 10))
 (segment (start 43.815 32.385) (end 34.09763 32.385) (width 0.6) (layer B.Cu) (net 10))
 (segment (start 34.09763 32.385) (end 33.02 32.385) (width 0.6) (layer B.Cu) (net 10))
 (segment (start 78.74 43.815) (end 76.99 43.815) (width 0.6) (layer B.Cu) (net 6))
 (segment (start 76.99 43.815) (end 74.295 41.12) (width 0.6) (layer B.Cu) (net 6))
 (segment (start 74.295 41.12) (end 74.295 39.908492) (width 0.6) (layer B.Cu) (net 6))
 (segment (start 74.295 39.908492) (end 74.295 38.495) (width 0.6) (layer B.Cu) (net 6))
 (segment (start 57.496 40.64) (end 55.88 40.64) (width 0.6) (layer B.Cu) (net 6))
 (segment (start 64.011752 40.64) (end 57.496 40.64) (width 0.6) (layer B.Cu) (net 6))
 (segment (start 71.33673 47.964978) (end 64.011752 40.64) (width 0.6) (layer B.Cu) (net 6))
 (segment (start 80.940022 47.964978) (end 71.33673 47.964978) (width 0.6) (layer B.Cu) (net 6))
 (segment (start 80.941989 47.963011) (end 80.940022 47.964978) (width 0.6) (layer B.Cu) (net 6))
 (segment (start 80.49 45.215) (end 80.49 45.50195) (width 0.6) (layer B.Cu) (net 6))
 (segment (start 80.49 45.50195) (end 80.941989 45.953939) (width 0.6) (layer B.Cu) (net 6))
 (segment (start 80.941989 45.953939) (end 80.941989 47.963011) (width 0.6) (layer B.Cu) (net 6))
 (segment (start 78.74 43.815) (end 79.09 43.815) (width 0.6) (layer B.Cu) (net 6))
 (segment (start 79.09 43.815) (end 80.49 45.215) (width 0.6) (layer B.Cu) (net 6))
 (segment (start 55.88 38.1) (end 55.88 40.64) (width 0.6) (layer B.Cu) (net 6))
 (segment (start 91.44 40.64) (end 97.155 40.64) (width 0.6) (layer B.Cu) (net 19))
 (segment (start 33.02 29.845) (end 38.1 29.845) (width 0.6) (layer B.Cu) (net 13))
 (segment (start 38.1 37.465) (end 38.1 40.005) (width 0.6) (layer B.Cu) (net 12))
 (segment (start 38.1 40.005) (end 36.83 41.275) (width 0.6) (layer B.Cu) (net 12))
 (segment (start 36.83 41.275) (end 33.02 41.275) (width 0.6) (layer B.Cu) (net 12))
 (segment (start 78.74 46.355) (end 76.835 46.355) (width 0.6) (layer B.Cu) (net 7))
 (segment (start 76.835 46.355) (end 71.755 41.275) (width 0.6) (layer B.Cu) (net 7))
 (segment (start 71.755 41.275) (end 71.755 36.195) (width 0.6) (layer B.Cu) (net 7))
 (segment (start 71.755 36.195) (end 74.295 33.655) (width 0.6) (layer B.Cu) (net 7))
 (segment (start 74.295 33.655) (end 74.295 29.21) (width 0.6) (layer B.Cu) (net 7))
 (segment (start 74.295 29.21) (end 75.565 27.94) (width 0.6) (layer B.Cu) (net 7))
 (segment (start 75.565 27.94) (end 77.47 27.94) (width 0.6) (layer B.Cu) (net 7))
 (segment (start 77.47 27.94) (end 77.47 22.86) (width 0.6) (layer B.Cu) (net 7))
 (segment (start 77.47 22.86) (end 78.74 21.59) (width 0.6) (layer B.Cu) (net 7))
 (segment (start 78.74 21.59) (end 80.01 21.59) (width 0.6) (layer B.Cu) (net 7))
 (segment (start 87.63 21.59) (end 92.71 21.59) (width 0.6) (layer B.Cu) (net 7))
 (segment (start 96.52 27.94) (end 97.155 28.575) (width 0.6) (layer B.Cu) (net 7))
 (segment (start 97.155 28.575) (end 97.155 35.56) (width 0.6) (layer B.Cu) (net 7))
 (segment (start 92.71 21.59) (end 93.345 22.225) (width 0.6) (layer B.Cu) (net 7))
 (segment (start 95.25 27.94) (end 96.52 27.94) (width 0.6) (layer B.Cu) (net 7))
 (segment (start 93.345 22.225) (end 93.345 26.035) (width 0.6) (layer B.Cu) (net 7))
 (segment (start 93.345 26.035) (end 95.25 27.94) (width 0.6) (layer B.Cu) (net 7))
 (segment (start 86.36 38.735) (end 86.36 34.925) (width 0.6) (layer B.Cu) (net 7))
 (segment (start 86.36 34.925) (end 85.09 33.655) (width 0.6) (layer B.Cu) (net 7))
 (segment (start 85.09 33.655) (end 85.09 27.94) (width 0.6) (layer B.Cu) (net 7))
 (segment (start 85.09 27.94) (end 86.36 26.67) (width 0.6) (layer B.Cu) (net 7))
 (segment (start 86.36 26.67) (end 86.36 22.86) (width 0.6) (layer B.Cu) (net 7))
 (segment (start 86.36 22.86) (end 87.63 21.59) (width 0.6) (layer B.Cu) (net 7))
 (segment (start 34.925 22.86) (end 34.925 25.4) (width 0.6) (layer B.Cu) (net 7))
 (segment (start 29.845 35.56) (end 33.02 38.735) (width 0.6) (layer B.Cu) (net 7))
 (segment (start 36.195 21.59) (end 34.925 22.86) (width 0.6) (layer B.Cu) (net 7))
 (segment (start 48.26 22.225) (end 47.625 21.59) (width 0.6) (layer B.Cu) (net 7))
 (segment (start 34.925 25.4) (end 33.655 26.67) (width 0.6) (layer B.Cu) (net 7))
 (segment (start 48.26 23.495) (end 48.26 22.225) (width 0.6) (layer B.Cu) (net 7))
 (segment (start 47.625 21.59) (end 36.195 21.59) (width 0.6) (layer B.Cu) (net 7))
 (segment (start 33.655 26.67) (end 31.115 26.67) (width 0.6) (layer B.Cu) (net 7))
 (segment (start 31.115 26.67) (end 29.845 27.94) (width 0.6) (layer B.Cu) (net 7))
 (segment (start 29.845 27.94) (end 29.845 35.56) (width 0.6) (layer B.Cu) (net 7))
 (segment (start 52.705 23.495) (end 52.705 22.225) (width 0.6) (layer B.Cu) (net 7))
 (segment (start 52.705 22.225) (end 53.34 21.59) (width 0.6) (layer B.Cu) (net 7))
 (segment (start 53.34 21.59) (end 68.370675 21.59) (width 0.6) (layer B.Cu) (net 7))
 (segment (start 68.370675 21.59) (end 80.01 21.59) (width 0.6) (layer B.Cu) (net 7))
 (segment (start 87.63 21.59) (end 80.01 21.59) (width 0.6) (layer B.Cu) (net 7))
 (segment (start 48.26 23.495) (end 52.705 23.495) (width 0.6) (layer B.Cu) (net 7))
 (segment (start 83.82 34.925) (end 83.82 23.495) (width 0.6) (layer B.Cu) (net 5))
 (segment (start 83.82 34.925) (end 83.82 44.165) (width 0.6) (layer B.Cu) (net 5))
 (segment (start 83.82 44.165) (end 86.01 46.355) (width 0.6) (layer B.Cu) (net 5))
 (segment (start 86.01 46.355) (end 86.36 46.355) (width 0.6) (layer B.Cu) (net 5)))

